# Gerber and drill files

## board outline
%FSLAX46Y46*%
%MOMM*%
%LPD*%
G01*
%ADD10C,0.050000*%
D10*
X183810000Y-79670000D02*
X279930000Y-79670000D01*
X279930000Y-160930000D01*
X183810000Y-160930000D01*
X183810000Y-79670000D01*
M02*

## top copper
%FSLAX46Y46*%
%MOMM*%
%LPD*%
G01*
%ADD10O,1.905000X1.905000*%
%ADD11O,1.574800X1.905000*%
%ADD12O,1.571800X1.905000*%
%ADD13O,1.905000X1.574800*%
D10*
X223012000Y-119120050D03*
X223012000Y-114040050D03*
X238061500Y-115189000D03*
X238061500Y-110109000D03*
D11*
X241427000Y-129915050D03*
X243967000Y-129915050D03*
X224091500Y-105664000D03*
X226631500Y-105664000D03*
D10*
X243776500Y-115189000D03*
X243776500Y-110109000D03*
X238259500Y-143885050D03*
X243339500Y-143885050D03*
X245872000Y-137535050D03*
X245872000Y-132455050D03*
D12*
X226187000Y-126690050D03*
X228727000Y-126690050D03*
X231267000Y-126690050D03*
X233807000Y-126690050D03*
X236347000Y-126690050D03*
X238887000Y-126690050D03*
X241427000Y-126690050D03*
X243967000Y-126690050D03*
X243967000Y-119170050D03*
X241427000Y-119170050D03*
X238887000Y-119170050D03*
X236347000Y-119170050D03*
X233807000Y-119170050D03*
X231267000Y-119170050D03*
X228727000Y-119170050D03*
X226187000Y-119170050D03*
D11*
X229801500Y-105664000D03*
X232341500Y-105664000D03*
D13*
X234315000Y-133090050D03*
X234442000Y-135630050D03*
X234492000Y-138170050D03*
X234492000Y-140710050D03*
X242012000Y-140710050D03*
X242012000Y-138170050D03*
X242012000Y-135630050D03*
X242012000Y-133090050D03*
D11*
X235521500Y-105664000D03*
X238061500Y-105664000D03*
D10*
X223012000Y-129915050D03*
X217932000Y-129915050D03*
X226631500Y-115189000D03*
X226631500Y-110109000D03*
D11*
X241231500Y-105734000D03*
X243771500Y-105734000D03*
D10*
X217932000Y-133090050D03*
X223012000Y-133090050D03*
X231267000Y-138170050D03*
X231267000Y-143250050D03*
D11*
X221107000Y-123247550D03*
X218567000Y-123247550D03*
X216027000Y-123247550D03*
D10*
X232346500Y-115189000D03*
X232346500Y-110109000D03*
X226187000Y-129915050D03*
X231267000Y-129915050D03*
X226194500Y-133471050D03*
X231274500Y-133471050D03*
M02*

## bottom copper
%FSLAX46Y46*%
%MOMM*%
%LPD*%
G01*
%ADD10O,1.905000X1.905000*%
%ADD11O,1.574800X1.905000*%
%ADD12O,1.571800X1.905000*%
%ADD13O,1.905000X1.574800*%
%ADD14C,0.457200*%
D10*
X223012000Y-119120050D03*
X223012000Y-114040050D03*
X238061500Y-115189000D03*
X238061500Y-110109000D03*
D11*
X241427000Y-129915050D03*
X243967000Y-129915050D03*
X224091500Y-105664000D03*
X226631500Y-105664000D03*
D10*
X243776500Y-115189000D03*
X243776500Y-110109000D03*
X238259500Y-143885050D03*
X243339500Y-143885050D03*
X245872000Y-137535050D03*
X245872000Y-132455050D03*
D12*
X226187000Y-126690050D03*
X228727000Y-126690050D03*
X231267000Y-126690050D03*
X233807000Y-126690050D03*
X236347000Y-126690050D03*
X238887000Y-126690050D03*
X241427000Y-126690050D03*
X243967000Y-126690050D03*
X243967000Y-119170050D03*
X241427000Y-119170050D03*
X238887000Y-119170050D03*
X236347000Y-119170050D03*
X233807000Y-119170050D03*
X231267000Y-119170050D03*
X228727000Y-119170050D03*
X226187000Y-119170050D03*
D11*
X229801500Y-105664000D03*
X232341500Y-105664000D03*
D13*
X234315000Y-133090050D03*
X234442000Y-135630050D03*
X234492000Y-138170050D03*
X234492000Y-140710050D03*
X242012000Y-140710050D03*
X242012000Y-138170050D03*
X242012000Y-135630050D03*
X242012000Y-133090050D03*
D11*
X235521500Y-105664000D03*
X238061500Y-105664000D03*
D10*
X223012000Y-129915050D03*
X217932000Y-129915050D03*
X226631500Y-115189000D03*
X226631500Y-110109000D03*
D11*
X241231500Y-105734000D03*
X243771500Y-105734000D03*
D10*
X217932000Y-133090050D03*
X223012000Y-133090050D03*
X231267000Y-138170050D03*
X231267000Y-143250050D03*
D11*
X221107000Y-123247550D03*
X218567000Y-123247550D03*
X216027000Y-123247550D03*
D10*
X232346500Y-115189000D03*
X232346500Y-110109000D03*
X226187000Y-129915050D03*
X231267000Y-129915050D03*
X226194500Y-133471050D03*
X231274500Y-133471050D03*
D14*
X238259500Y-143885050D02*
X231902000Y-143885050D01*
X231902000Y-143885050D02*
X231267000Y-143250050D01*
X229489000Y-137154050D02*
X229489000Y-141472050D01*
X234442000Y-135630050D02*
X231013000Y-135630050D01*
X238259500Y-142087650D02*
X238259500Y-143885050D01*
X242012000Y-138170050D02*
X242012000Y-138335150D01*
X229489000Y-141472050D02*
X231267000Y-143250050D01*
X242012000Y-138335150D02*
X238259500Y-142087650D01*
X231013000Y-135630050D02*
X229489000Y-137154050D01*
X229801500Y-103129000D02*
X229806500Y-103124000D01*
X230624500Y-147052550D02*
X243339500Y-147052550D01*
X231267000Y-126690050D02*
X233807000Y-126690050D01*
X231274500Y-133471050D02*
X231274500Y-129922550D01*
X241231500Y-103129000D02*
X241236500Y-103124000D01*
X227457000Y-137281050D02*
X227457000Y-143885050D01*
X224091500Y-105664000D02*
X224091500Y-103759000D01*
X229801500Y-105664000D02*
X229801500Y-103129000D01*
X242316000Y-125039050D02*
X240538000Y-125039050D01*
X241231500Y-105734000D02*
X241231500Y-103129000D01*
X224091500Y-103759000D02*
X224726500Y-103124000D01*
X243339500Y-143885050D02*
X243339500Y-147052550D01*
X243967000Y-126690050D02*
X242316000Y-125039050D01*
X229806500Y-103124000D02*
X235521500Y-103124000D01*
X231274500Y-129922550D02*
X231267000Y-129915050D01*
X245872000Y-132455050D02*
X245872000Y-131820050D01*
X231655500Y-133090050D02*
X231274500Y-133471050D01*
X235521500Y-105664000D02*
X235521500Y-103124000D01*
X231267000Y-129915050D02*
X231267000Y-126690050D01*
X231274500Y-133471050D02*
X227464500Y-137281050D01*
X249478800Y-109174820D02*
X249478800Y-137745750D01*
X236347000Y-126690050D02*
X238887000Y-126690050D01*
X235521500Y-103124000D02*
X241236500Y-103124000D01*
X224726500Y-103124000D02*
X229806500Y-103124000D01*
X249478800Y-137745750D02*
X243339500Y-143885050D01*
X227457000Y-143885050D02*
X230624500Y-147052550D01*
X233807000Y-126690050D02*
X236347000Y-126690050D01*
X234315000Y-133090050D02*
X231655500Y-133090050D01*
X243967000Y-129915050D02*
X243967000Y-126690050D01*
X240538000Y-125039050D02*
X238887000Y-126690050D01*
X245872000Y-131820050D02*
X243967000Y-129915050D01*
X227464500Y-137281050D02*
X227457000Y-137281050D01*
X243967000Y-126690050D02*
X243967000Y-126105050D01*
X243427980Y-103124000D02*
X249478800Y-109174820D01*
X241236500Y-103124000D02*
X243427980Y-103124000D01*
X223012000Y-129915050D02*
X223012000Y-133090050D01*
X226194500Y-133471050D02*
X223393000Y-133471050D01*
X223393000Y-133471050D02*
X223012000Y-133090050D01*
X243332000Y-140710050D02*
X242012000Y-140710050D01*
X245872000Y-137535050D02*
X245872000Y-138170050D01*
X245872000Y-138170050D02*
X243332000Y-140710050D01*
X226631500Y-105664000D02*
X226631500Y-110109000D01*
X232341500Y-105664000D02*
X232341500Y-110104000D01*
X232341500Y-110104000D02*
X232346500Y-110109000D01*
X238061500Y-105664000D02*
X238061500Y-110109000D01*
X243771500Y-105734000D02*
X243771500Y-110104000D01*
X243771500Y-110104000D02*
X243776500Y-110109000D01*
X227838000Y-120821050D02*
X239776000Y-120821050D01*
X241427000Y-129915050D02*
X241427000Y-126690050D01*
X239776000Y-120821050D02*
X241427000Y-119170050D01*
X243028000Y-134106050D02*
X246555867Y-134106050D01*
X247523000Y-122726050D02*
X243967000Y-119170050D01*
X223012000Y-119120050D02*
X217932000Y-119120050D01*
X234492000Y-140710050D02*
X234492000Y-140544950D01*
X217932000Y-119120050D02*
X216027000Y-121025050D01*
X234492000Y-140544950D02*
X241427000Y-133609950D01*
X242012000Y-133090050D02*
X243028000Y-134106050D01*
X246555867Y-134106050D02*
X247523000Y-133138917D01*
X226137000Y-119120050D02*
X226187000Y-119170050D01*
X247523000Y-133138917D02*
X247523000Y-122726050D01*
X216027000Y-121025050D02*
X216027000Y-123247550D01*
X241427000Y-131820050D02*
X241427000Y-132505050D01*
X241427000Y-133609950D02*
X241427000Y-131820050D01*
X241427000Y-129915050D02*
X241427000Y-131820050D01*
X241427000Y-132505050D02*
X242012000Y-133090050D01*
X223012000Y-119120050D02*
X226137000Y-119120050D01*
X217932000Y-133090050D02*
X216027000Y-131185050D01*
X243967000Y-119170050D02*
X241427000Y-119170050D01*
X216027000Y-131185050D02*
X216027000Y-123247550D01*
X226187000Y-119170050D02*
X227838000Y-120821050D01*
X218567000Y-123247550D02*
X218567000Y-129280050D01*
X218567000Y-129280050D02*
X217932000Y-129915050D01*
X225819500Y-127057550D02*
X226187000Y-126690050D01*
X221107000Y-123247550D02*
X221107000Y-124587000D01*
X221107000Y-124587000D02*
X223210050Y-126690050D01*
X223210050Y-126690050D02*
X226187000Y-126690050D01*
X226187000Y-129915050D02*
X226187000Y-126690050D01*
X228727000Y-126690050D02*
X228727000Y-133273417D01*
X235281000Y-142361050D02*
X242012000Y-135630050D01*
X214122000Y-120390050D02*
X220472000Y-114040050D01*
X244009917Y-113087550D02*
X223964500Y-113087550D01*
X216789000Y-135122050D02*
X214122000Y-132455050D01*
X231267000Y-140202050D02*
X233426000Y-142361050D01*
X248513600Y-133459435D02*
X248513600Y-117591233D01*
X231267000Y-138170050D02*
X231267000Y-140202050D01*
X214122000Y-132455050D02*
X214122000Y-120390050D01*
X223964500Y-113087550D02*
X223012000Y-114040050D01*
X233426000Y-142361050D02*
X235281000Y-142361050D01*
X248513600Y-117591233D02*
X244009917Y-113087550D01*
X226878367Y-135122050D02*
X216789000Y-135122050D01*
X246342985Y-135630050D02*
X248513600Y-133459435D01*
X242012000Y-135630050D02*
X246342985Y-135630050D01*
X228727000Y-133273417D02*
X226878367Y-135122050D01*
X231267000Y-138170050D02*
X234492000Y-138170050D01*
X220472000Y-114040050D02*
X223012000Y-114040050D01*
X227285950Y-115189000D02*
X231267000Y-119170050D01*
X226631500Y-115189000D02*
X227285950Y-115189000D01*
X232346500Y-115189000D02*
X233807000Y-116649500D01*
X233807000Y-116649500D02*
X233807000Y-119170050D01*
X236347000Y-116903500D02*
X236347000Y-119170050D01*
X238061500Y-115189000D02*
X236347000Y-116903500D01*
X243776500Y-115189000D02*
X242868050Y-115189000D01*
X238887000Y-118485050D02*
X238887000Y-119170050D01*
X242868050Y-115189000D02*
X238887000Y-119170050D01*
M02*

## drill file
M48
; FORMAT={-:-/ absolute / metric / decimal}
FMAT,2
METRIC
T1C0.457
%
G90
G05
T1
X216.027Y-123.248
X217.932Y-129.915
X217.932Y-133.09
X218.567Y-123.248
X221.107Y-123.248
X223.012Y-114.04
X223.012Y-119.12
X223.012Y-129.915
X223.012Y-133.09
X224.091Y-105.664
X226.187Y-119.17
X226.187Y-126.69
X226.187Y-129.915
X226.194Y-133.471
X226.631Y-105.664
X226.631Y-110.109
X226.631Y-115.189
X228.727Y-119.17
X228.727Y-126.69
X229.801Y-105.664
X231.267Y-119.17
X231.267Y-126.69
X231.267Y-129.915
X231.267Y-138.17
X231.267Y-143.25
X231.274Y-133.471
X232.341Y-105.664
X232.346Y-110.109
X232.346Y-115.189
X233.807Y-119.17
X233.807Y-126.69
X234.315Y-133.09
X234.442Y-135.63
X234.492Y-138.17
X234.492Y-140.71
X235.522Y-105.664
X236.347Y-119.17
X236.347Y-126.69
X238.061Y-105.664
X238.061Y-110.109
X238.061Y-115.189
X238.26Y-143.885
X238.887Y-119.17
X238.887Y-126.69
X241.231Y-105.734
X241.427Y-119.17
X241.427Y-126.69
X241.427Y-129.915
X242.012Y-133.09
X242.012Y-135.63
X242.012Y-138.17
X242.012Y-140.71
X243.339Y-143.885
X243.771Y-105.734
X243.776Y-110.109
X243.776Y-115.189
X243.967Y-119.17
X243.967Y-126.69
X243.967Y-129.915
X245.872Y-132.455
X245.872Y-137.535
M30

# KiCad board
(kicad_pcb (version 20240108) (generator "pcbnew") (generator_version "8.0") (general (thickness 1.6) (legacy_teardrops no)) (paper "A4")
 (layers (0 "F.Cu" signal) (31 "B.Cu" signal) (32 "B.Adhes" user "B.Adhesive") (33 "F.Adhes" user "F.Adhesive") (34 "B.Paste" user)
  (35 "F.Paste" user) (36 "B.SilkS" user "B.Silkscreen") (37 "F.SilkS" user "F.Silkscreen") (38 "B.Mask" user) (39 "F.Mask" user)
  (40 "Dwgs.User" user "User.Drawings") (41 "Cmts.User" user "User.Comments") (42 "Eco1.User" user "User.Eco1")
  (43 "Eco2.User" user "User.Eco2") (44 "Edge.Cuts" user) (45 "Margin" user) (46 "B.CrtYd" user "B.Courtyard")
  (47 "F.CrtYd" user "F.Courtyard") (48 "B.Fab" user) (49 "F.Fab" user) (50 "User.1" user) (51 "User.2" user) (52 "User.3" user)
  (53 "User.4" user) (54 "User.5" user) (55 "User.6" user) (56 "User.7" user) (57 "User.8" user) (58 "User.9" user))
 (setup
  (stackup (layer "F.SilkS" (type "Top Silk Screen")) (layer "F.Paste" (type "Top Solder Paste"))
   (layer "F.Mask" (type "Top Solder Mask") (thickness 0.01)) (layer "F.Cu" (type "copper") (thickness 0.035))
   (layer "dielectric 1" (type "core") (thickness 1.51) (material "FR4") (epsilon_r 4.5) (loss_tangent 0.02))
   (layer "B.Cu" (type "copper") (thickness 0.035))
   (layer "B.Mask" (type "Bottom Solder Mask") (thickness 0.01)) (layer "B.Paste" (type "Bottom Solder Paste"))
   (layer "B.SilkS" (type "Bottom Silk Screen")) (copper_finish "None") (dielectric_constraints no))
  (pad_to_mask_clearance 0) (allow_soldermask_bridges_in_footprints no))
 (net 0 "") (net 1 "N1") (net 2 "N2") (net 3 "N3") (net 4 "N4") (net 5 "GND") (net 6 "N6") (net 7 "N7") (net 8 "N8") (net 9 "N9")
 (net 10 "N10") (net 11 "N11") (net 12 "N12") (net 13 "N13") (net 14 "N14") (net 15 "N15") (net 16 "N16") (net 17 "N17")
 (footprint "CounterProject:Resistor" (layer "F.Cu") (at 223.012 119.12005 90)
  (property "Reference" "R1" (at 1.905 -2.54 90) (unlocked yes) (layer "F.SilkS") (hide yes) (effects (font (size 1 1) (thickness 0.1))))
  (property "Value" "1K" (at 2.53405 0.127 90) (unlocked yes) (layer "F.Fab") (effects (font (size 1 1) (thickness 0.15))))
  (pad "1" thru_hole oval (at 0 0 90) (size 1.905 1.905) (drill 0.4572) (layers "*.Cu" "*.Mask") (remove_unused_layers no) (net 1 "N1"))
  (pad "2" thru_hole oval (at 5.08 0 90) (size 1.905 1.905) (drill 0.4572) (layers "*.Cu" "*.Mask") (remove_unused_layers no) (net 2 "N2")))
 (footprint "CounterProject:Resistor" (layer "F.Cu") (at 238.0615 115.189 90)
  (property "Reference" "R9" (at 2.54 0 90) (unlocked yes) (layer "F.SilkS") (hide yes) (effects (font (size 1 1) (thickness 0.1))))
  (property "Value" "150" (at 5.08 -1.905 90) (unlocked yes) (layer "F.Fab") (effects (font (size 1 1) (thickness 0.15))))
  (pad "1" thru_hole oval (at 0 0 90) (size 1.905 1.905) (drill 0.4572) (layers "*.Cu" "*.Mask") (remove_unused_layers no) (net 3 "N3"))
  (pad "2" thru_hole oval (at 5.08 0 90) (size 1.905 1.905) (drill 0.4572) (layers "*.Cu" "*.Mask") (remove_unused_layers no) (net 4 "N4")))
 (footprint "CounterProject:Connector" (layer "F.Cu") (at 241.427 129.91505)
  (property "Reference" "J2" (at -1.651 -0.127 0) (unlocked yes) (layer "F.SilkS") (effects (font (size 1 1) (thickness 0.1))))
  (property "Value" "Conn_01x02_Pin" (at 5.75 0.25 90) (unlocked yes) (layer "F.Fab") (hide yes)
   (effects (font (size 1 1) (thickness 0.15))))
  (pad "1" thru_hole oval (at 0 0) (size 1.5748 1.905) (drill 0.4572) (layers "*.Cu" "*.Mask") (remove_unused_layers no) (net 1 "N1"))
  (pad "2" thru_hole oval (at 2.54 0) (size 1.5748 1.905) (drill 0.4572) (layers "*.Cu" "*.Mask") (remove_unused_layers no) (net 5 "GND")))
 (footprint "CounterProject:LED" (layer "F.Cu") (at 224.0915 105.664)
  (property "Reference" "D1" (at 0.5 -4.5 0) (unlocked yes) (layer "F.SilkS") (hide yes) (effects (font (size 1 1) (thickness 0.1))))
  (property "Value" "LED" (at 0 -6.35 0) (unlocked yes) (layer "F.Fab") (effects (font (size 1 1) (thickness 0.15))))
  (pad "1" thru_hole oval (at 0 0) (size 1.5748 1.905) (drill 0.4572) (layers "*.Cu" "*.Mask") (remove_unused_layers no) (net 5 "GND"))
  (pad "2" thru_hole oval (at 2.54 0) (size 1.5748 1.905) (drill 0.4572) (layers "*.Cu" "*.Mask") (remove_unused_layers no) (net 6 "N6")))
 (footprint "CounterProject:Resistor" (layer "F.Cu") (at 243.7765 115.189 90)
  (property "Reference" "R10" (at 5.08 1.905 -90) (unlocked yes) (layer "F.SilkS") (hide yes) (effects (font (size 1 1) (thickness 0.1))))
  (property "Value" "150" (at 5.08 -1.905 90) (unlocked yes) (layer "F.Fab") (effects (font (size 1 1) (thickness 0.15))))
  (pad "1" thru_hole oval (at 0 0 90) (size 1.905 1.905) (drill 0.4572) (layers "*.Cu" "*.Mask") (remove_unused_layers no) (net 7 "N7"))
  (pad "2" thru_hole oval (at 5.08 0 90) (size 1.905 1.905) (drill 0.4572) (layers "*.Cu" "*.Mask") (remove_unused_layers no) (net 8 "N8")))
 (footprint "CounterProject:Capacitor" (layer "F.Cu") (at 238.2595 143.88505)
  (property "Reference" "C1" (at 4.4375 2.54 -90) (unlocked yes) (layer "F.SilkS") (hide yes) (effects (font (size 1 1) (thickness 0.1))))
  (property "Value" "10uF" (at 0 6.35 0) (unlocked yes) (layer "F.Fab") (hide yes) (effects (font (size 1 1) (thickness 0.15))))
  (pad "1" thru_hole oval (at 0 0) (size 1.905 1.905) (drill 0.4572) (layers "*.Cu" "*.Mask") (remove_unused_layers no) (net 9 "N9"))
  (pad "2" thru_hole oval (at 5.08 0) (size 1.905 1.905) (drill 0.4572) (layers "*.Cu" "*.Mask") (remove_unused_layers no) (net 5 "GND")))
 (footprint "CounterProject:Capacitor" (layer "F.Cu") (at 245.872 137.53505 90)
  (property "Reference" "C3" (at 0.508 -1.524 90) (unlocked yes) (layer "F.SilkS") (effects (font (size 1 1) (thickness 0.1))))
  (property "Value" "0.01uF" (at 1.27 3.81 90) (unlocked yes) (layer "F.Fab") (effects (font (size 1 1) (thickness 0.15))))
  (pad "1" thru_hole oval (at 0 0 90) (size 1.905 1.905) (drill 0.4572) (layers "*.Cu" "*.Mask") (remove_unused_layers no) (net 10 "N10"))
  (pad "2" thru_hole oval (at 5.08 0 90) (size 1.905 1.905) (drill 0.4572) (layers "*.Cu" "*.Mask") (remove_unused_layers no) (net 5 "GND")))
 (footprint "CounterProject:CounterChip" (layer "F.Cu") (at 226.1616 126.66465)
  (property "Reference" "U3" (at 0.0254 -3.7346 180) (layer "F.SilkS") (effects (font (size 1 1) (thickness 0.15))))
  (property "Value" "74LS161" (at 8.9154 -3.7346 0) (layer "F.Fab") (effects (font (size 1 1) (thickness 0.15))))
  (pad "1" thru_hole oval (at 0.0254 0.0254) (size 1.5718 1.905) (drill 0.4572) (layers "*.Cu" "*.Mask") (remove_unused_layers no)
   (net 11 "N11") (thermal_bridge_angle 45))
  (pad "2" thru_hole oval (at 2.5654 0.0254) (size 1.5718 1.905) (drill 0.4572) (layers "*.Cu" "*.Mask") (remove_unused_layers no)
   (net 2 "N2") (thermal_bridge_angle 45))
  (pad "3" thru_hole oval (at 5.1054 0.0254) (size 1.5718 1.905) (drill 0.4572) (layers "*.Cu" "*.Mask") (remove_unused_layers no)
   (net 5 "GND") (thermal_bridge_angle 45))
  (pad "4" thru_hole oval (at 7.6454 0.0254) (size 1.5718 1.905) (drill 0.4572) (layers "*.Cu" "*.Mask") (remove_unused_layers no)
   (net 5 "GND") (thermal_bridge_angle 45))
  (pad "5" thru_hole oval (at 10.1854 0.0254) (size 1.5718 1.905) (drill 0.4572) (layers "*.Cu" "*.Mask") (remove_unused_layers no)
   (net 5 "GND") (thermal_bridge_angle 45))
  (pad "6" thru_hole oval (at 12.7254 0.0254) (size 1.5718 1.905) (drill 0.4572) (layers "*.Cu" "*.Mask") (remove_unused_layers no)
   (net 5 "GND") (thermal_bridge_angle 45))
  (pad "7" thru_hole oval (at 15.2654 0.0254) (size 1.5718 1.905) (drill 0.4572) (layers "*.Cu" "*.Mask") (remove_unused_layers no)
   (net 1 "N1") (thermal_bridge_angle 45))
  (pad "8" thru_hole oval (at 17.8054 0.0254) (size 1.5718 1.905) (drill 0.4572) (layers "*.Cu" "*.Mask") (remove_unused_layers no)
   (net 5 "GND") (thermal_bridge_angle 45))
  (pad "9" thru_hole oval (at 17.8054 -7.4946) (size 1.5718 1.905) (drill 0.4572) (layers "*.Cu" "*.Mask") (remove_unused_layers no)
   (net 1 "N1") (thermal_bridge_angle 45))
  (pad "10" thru_hole oval (at 15.2654 -7.4946) (size 1.5718 1.905) (drill 0.4572) (layers "*.Cu" "*.Mask") (remove_unused_layers no)
   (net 1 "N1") (thermal_bridge_angle 45))
  (pad "11" thru_hole oval (at 12.7254 -7.4946) (size 1.5718 1.905) (drill 0.4572) (layers "*.Cu" "*.Mask") (remove_unused_layers no)
   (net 7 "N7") (thermal_bridge_angle 45))
  (pad "12" thru_hole oval (at 10.1854 -7.4946) (size 1.5718 1.905) (drill 0.4572) (layers "*.Cu" "*.Mask") (remove_unused_layers no)
   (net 3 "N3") (thermal_bridge_angle 45))
  (pad "13" thru_hole oval (at 7.6454 -7.4946) (size 1.5718 1.905) (drill 0.4572) (layers "*.Cu" "*.Mask") (remove_unused_layers no)
   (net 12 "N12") (thermal_bridge_angle 45))
  (pad "14" thru_hole oval (at 5.1054 -7.4946) (size 1.5718 1.905) (drill 0.4572) (layers "*.Cu" "*.Mask") (remove_unused_layers no)
   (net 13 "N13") (thermal_bridge_angle 45))
  (pad "15" thru_hole oval (at 2.5654 -7.4946) (size 1.5718 1.905) (drill 0.4572) (layers "*.Cu" "*.Mask") (remove_unused_layers no)
   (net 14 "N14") (thermal_bridge_angle 45))
  (pad "16" thru_hole oval (at 0.0254 -7.4946) (size 1.5718 1.905) (drill 0.4572) (layers "*.Cu" "*.Mask") (remove_unused_layers no)
   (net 1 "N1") (thermal_bridge_angle 45)))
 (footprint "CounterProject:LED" (layer "F.Cu") (at 229.8015 105.664)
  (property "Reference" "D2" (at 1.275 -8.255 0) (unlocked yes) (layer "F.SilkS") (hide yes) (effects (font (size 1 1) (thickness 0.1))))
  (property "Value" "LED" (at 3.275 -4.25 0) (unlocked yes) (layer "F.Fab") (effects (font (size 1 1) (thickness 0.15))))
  (pad "1" thru_hole oval (at 0 0) (size 1.5748 1.905) (drill 0.4572) (layers "*.Cu" "*.Mask") (remove_unused_layers no) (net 5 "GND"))
  (pad "2" thru_hole oval (at 2.54 0) (size 1.5748 1.905) (drill 0.4572) (layers "*.Cu" "*.Mask") (remove_unused_layers no) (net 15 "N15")))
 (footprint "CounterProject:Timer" (layer "F.Cu") (at 234.315 133.09005 -90)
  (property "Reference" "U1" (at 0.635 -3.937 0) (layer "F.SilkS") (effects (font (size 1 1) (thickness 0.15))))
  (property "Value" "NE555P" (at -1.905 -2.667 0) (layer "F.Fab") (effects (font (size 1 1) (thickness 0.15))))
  (pad "1" thru_hole oval (at 0 0 270) (size 1.5748 1.905) (drill 0.4572) (layers "*.Cu" "*.Mask") (remove_unused_layers no) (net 5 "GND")
   (thermal_bridge_angle 45))
  (pad "2" thru_hole oval (at 2.54 -0.127 270) (size 1.5748 1.905) (drill 0.4572) (layers "*.Cu" "*.Mask") (remove_unused_layers no)
   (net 9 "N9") (thermal_bridge_angle 45))
  (pad "3" thru_hole oval (at 5.08 -0.177 270) (size 1.5748 1.905) (drill 0.4572) (layers "*.Cu" "*.Mask") (remove_unused_layers no)
   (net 2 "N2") (thermal_bridge_angle 45))
  (pad "4" thru_hole oval (at 7.62 -0.177 270) (size 1.5748 1.905) (drill 0.4572) (layers "*.Cu" "*.Mask") (remove_unused_layers no)
   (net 1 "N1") (thermal_bridge_angle 45))
  (pad "5" thru_hole oval (at 7.62 -7.697 270) (size 1.5748 1.905) (drill 0.4572) (layers "*.Cu" "*.Mask") (remove_unused_layers no)
   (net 10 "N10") (thermal_bridge_angle 45))
  (pad "6" thru_hole oval (at 5.08 -7.697 270) (size 1.5748 1.905) (drill 0.4572) (layers "*.Cu" "*.Mask") (remove_unused_layers no)
   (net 9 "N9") (thermal_bridge_angle 45))
  (pad "7" thru_hole oval (at 2.54 -7.697 270) (size 1.5748 1.905) (drill 0.4572) (layers "*.Cu" "*.Mask") (remove_unused_layers no)
   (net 2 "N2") (thermal_bridge_angle 45))
  (pad "8" thru_hole oval (at 0 -7.697 270) (size 1.5748 1.905) (drill 0.4572) (layers "*.Cu" "*.Mask") (remove_unused_layers no)
   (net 1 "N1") (thermal_bridge_angle 45)))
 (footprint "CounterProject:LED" (layer "F.Cu") (at 235.5215 105.664)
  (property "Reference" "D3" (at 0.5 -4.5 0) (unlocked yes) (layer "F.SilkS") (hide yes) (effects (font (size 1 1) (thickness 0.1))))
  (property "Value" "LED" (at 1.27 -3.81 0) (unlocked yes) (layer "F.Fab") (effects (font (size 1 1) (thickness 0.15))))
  (pad "1" thru_hole oval (at 0 0) (size 1.5748 1.905) (drill 0.4572) (layers "*.Cu" "*.Mask") (remove_unused_layers no) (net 5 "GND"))
  (pad "2" thru_hole oval (at 2.54 0) (size 1.5748 1.905) (drill 0.4572) (layers "*.Cu" "*.Mask") (remove_unused_layers no) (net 4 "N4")))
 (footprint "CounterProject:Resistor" (layer "F.Cu") (at 223.012 129.91505 180)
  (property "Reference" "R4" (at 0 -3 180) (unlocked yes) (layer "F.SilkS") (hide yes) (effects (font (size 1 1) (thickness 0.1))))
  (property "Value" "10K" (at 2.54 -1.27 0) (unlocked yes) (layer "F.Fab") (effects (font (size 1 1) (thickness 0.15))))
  (pad "1" thru_hole oval (at 0 0 180) (size 1.905 1.905) (drill 0.4572) (layers "*.Cu" "*.Mask") (remove_unused_layers no) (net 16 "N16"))
  (pad "2" thru_hole oval (at 5.08 0 180) (size 1.905 1.905) (drill 0.4572) (layers "*.Cu" "*.Mask") (remove_unused_layers no)
   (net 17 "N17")))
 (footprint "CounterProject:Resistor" (layer "F.Cu") (at 226.6315 115.189 90)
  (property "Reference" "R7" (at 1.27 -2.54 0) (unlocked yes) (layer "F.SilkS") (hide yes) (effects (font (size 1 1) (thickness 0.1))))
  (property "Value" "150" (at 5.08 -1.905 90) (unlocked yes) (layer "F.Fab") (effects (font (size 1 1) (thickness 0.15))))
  (pad "1" thru_hole oval (at 0 0 90) (size 1.905 1.905) (drill 0.4572) (layers "*.Cu" "*.Mask") (remove_unused_layers no) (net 13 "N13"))
  (pad "2" thru_hole oval (at 5.08 0 90) (size 1.905 1.905) (drill 0.4572) (layers "*.Cu" "*.Mask") (remove_unused_layers no) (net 6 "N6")))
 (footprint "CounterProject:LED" (layer "F.Cu") (at 241.2315 105.734)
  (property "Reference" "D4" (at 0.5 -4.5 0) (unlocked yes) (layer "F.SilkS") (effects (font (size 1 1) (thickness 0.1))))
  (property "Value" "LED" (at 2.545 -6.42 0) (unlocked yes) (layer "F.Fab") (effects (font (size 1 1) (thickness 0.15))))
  (pad "1" thru_hole oval (at 0 0) (size 1.5748 1.905) (drill 0.4572) (layers "*.Cu" "*.Mask") (remove_unused_layers no) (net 5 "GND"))
  (pad "2" thru_hole oval (at 2.54 0) (size 1.5748 1.905) (drill 0.4572) (layers "*.Cu" "*.Mask") (remove_unused_layers no) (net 8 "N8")))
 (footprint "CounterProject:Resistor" (layer "F.Cu") (at 217.932 133.09005)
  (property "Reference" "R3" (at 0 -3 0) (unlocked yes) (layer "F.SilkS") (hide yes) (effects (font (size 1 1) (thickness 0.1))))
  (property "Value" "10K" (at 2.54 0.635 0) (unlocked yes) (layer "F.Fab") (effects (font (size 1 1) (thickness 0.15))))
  (pad "1" thru_hole oval (at 0 0) (size 1.905 1.905) (drill 0.4572) (layers "*.Cu" "*.Mask") (remove_unused_layers no) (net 1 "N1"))
  (pad "2" thru_hole oval (at 5.08 0) (size 1.905 1.905) (drill 0.4572) (layers "*.Cu" "*.Mask") (remove_unused_layers no) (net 16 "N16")))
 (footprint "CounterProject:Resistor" (layer "F.Cu") (at 231.267 138.17005 -90)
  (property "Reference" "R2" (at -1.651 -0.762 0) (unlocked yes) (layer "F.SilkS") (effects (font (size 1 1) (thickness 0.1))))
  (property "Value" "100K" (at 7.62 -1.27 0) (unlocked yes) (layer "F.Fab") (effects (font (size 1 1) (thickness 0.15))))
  (pad "1" thru_hole oval (at 0 0 270) (size 1.905 1.905) (drill 0.4572) (layers "*.Cu" "*.Mask") (remove_unused_layers no) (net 2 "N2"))
  (pad "2" thru_hole oval (at 5.08 0 270) (size 1.905 1.905) (drill 0.4572) (layers "*.Cu" "*.Mask") (remove_unused_layers no) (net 9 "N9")))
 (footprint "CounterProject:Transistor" (layer "F.Cu") (at 221.107 123.24755 180)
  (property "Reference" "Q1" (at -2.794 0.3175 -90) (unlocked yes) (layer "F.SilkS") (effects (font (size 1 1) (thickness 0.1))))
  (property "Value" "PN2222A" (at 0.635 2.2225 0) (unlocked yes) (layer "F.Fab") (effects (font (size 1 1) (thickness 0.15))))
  (pad "1" thru_hole oval (at 0 0 180) (size 1.5748 1.905) (drill 0.4572) (layers "*.Cu" "*.Mask") (remove_unused_layers no) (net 11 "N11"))
  (pad "2" thru_hole oval (at 2.54 0 180) (size 1.5748 1.905) (drill 0.4572) (layers "*.Cu" "*.Mask") (remove_unused_layers no)
   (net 17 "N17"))
  (pad "3" thru_hole oval (at 5.08 0 180) (size 1.5748 1.905) (drill 0.4572) (layers "*.Cu" "*.Mask") (remove_unused_layers no) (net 1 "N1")))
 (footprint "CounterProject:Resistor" (layer "F.Cu") (at 232.3465 115.189 90)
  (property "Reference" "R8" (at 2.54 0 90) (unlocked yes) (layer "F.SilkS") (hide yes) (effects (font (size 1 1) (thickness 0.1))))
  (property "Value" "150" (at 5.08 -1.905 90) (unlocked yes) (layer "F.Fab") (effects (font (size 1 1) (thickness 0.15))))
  (pad "1" thru_hole oval (at 0 0 90) (size 1.905 1.905) (drill 0.4572) (layers "*.Cu" "*.Mask") (remove_unused_layers no) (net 12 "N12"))
  (pad "2" thru_hole oval (at 5.08 0 90) (size 1.905 1.905) (drill 0.4572) (layers "*.Cu" "*.Mask") (remove_unused_layers no) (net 15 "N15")))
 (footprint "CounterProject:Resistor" (layer "F.Cu") (at 226.187 129.91505)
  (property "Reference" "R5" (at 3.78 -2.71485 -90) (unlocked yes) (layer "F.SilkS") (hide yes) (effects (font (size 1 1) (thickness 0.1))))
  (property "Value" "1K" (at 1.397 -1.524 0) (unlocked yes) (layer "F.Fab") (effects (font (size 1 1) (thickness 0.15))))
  (pad "1" thru_hole oval (at 0 0) (size 1.905 1.905) (drill 0.4572) (layers "*.Cu" "*.Mask") (remove_unused_layers no) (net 11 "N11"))
  (pad "2" thru_hole oval (at 5.08 0) (size 1.905 1.905) (drill 0.4572) (layers "*.Cu" "*.Mask") (remove_unused_layers no) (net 5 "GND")))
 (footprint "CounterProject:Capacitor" (layer "F.Cu") (at 226.1945 133.47105)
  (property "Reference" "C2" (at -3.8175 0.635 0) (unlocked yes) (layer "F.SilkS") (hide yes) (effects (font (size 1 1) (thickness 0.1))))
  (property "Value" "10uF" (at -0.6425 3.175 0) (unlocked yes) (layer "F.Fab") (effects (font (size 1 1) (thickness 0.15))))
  (pad "1" thru_hole oval (at 0 0) (size 1.905 1.905) (drill 0.4572) (layers "*.Cu" "*.Mask") (remove_unused_layers no) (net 16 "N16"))
  (pad "2" thru_hole oval (at 5.08 0) (size 1.905 1.905) (drill 0.4572) (layers "*.Cu" "*.Mask") (remove_unused_layers no) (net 5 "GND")))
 (gr_rect (start 183.81 79.67) (end 279.93 160.93) (stroke (width 0.05) (type default)) (fill none) (layer "Edge.Cuts"))
 (segment (start 238.2595 143.88505) (end 231.902 143.88505) (width 0.4572) (layer "B.Cu") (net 9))
 (segment (start 231.902 143.88505) (end 231.267 143.25005) (width 0.4572) (layer "B.Cu") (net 9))
 (segment (start 229.489 137.15405) (end 229.489 141.47205) (width 0.4572) (layer "B.Cu") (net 9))
 (segment (start 234.442 135.63005) (end 231.013 135.63005) (width 0.4572) (layer "B.Cu") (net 9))
 (segment (start 238.2595 142.08765) (end 238.2595 143.88505) (width 0.4572) (layer "B.Cu") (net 9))
 (segment (start 242.012 138.17005) (end 242.012 138.33515) (width 0.4572) (layer "B.Cu") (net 9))
 (segment (start 229.489 141.47205) (end 231.267 143.25005) (width 0.4572) (layer "B.Cu") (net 9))
 (segment (start 242.012 138.33515) (end 238.2595 142.08765) (width 0.4572) (layer "B.Cu") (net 9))
 (segment (start 231.013 135.63005) (end 229.489 137.15405) (width 0.4572) (layer "B.Cu") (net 9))
 (segment (start 229.8015 103.129) (end 229.8065 103.124) (width 0.4572) (layer "B.Cu") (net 5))
 (segment (start 230.6245 147.05255) (end 243.3395 147.05255) (width 0.4572) (layer "B.Cu") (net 5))
 (segment (start 231.267 126.69005) (end 233.807 126.69005) (width 0.4572) (layer "B.Cu") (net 5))
 (segment (start 231.2745 133.47105) (end 231.2745 129.92255) (width 0.4572) (layer "B.Cu") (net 5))
 (segment (start 241.2315 103.129) (end 241.2365 103.124) (width 0.4572) (layer "B.Cu") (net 5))
 (segment (start 227.457 137.28105) (end 227.457 143.88505) (width 0.4572) (layer "B.Cu") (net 5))
 (segment (start 224.0915 105.664) (end 224.0915 103.759) (width 0.4572) (layer "B.Cu") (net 5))
 (segment (start 229.8015 105.664) (end 229.8015 103.129) (width 0.4572) (layer "B.Cu") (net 5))
 (segment (start 242.316 125.03905) (end 240.538 125.03905) (width 0.4572) (layer "B.Cu") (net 5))
 (segment (start 241.2315 105.734) (end 241.2315 103.129) (width 0.4572) (layer "B.Cu") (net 5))
 (segment (start 224.0915 103.759) (end 224.7265 103.124) (width 0.4572) (layer "B.Cu") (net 5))
 (segment (start 243.3395 143.88505) (end 243.3395 147.05255) (width 0.4572) (layer "B.Cu") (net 5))
 (segment (start 243.967 126.69005) (end 242.316 125.03905) (width 0.4572) (layer "B.Cu") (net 5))
 (segment (start 229.8065 103.124) (end 235.5215 103.124) (width 0.4572) (layer "B.Cu") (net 5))
 (segment (start 231.2745 129.92255) (end 231.267 129.91505) (width 0.4572) (layer "B.Cu") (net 5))
 (segment (start 245.872 132.45505) (end 245.872 131.82005) (width 0.4572) (layer "B.Cu") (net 5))
 (segment (start 231.6555 133.09005) (end 231.2745 133.47105) (width 0.4572) (layer "B.Cu") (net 5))
 (segment (start 235.5215 105.664) (end 235.5215 103.124) (width 0.4572) (layer "B.Cu") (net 5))
 (segment (start 231.267 129.91505) (end 231.267 126.69005) (width 0.4572) (layer "B.Cu") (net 5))
 (segment (start 231.2745 133.47105) (end 227.4645 137.28105) (width 0.4572) (layer "B.Cu") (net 5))
 (segment (start 249.4788 109.17482) (end 249.4788 137.74575) (width 0.4572) (layer "B.Cu") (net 5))
 (segment (start 236.347 126.69005) (end 238.887 126.69005) (width 0.4572) (layer "B.Cu") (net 5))
 (segment (start 235.5215 103.124) (end 241.2365 103.124) (width 0.4572) (layer "B.Cu") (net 5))
 (segment (start 224.7265 103.124) (end 229.8065 103.124) (width 0.4572) (layer "B.Cu") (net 5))
 (segment (start 249.4788 137.74575) (end 243.3395 143.88505) (width 0.4572) (layer "B.Cu") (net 5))
 (segment (start 227.457 143.88505) (end 230.6245 147.05255) (width 0.4572) (layer "B.Cu") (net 5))
 (segment (start 233.807 126.69005) (end 236.347 126.69005) (width 0.4572) (layer "B.Cu") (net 5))
 (segment (start 234.315 133.09005) (end 231.6555 133.09005) (width 0.4572) (layer "B.Cu") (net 5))
 (segment (start 243.967 129.91505) (end 243.967 126.69005) (width 0.4572) (layer "B.Cu") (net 5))
 (segment (start 240.538 125.03905) (end 238.887 126.69005) (width 0.4572) (layer "B.Cu") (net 5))
 (segment (start 245.872 131.82005) (end 243.967 129.91505) (width 0.4572) (layer "B.Cu") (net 5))
 (segment (start 227.4645 137.28105) (end 227.457 137.28105) (width 0.4572) (layer "B.Cu") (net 5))
 (segment (start 243.967 126.69005) (end 243.967 126.10505) (width 0.4572) (layer "B.Cu") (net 5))
 (segment (start 243.42798 103.124) (end 249.4788 109.17482) (width 0.4572) (layer "B.Cu") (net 5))
 (segment (start 241.2365 103.124) (end 243.42798 103.124) (width 0.4572) (layer "B.Cu") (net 5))
 (segment (start 223.012 129.91505) (end 223.012 133.09005) (width 0.4572) (layer "B.Cu") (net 16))
 (segment (start 226.1945 133.47105) (end 223.393 133.47105) (width 0.4572) (layer "B.Cu") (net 16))
 (segment (start 223.393 133.47105) (end 223.012 133.09005) (width 0.4572) (layer "B.Cu") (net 16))
 (segment (start 243.332 140.71005) (end 242.012 140.71005) (width 0.4572) (layer "B.Cu") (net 10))
 (segment (start 245.872 137.53505) (end 245.872 138.17005) (width 0.4572) (layer "B.Cu") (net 10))
 (segment (start 245.872 138.17005) (end 243.332 140.71005) (width 0.4572) (layer "B.Cu") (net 10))
 (segment (start 226.6315 105.664) (end 226.6315 110.109) (width 0.4572) (layer "B.Cu") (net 6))
 (segment (start 232.3415 105.664) (end 232.3415 110.104) (width 0.4572) (layer "B.Cu") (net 15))
 (segment (start 232.3415 110.104) (end 232.3465 110.109) (width 0.4572) (layer "B.Cu") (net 15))
 (segment (start 238.0615 105.664) (end 238.0615 110.109) (width 0.4572) (layer "B.Cu") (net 4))
 (segment (start 243.7715 105.734) (end 243.7715 110.104) (width 0.4572) (layer "B.Cu") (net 8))
 (segment (start 243.7715 110.104) (end 243.7765 110.109) (width 0.4572) (layer "B.Cu") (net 8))
 (segment (start 227.838 120.82105) (end 239.776 120.82105) (width 0.4572) (layer "B.Cu") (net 1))
 (segment (start 241.427 129.91505) (end 241.427 126.69005) (width 0.4572) (layer "B.Cu") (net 1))
 (segment (start 239.776 120.82105) (end 241.427 119.17005) (width 0.4572) (layer "B.Cu") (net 1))
 (segment (start 243.028 134.10605) (end 246.555867 134.10605) (width 0.4572) (layer "B.Cu") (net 1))
 (segment (start 247.523 122.72605) (end 243.967 119.17005) (width 0.4572) (layer "B.Cu") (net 1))
 (segment (start 223.012 119.12005) (end 217.932 119.12005) (width 0.4572) (layer "B.Cu") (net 1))
 (segment (start 234.492 140.71005) (end 234.492 140.54495) (width 0.4572) (layer "B.Cu") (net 1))
 (segment (start 217.932 119.12005) (end 216.027 121.02505) (width 0.4572) (layer "B.Cu") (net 1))
 (segment (start 234.492 140.54495) (end 241.427 133.60995) (width 0.4572) (layer "B.Cu") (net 1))
 (segment (start 242.012 133.09005) (end 243.028 134.10605) (width 0.4572) (layer "B.Cu") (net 1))
 (segment (start 246.555867 134.10605) (end 247.523 133.138917) (width 0.4572) (layer "B.Cu") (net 1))
 (segment (start 226.137 119.12005) (end 226.187 119.17005) (width 0.4572) (layer "B.Cu") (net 1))
 (segment (start 247.523 133.138917) (end 247.523 122.72605) (width 0.4572) (layer "B.Cu") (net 1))
 (segment (start 216.027 121.02505) (end 216.027 123.24755) (width 0.4572) (layer "B.Cu") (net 1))
 (segment (start 241.427 131.82005) (end 241.427 132.50505) (width 0.4572) (layer "B.Cu") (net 1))
 (segment (start 241.427 133.60995) (end 241.427 131.82005) (width 0.4572) (layer "B.Cu") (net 1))
 (segment (start 241.427 129.91505) (end 241.427 131.82005) (width 0.4572) (layer "B.Cu") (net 1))
 (segment (start 241.427 132.50505) (end 242.012 133.09005) (width 0.4572) (layer "B.Cu") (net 1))
 (segment (start 223.012 119.12005) (end 226.137 119.12005) (width 0.4572) (layer "B.Cu") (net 1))
 (segment (start 217.932 133.09005) (end 216.027 131.18505) (width 0.4572) (layer "B.Cu") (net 1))
 (segment (start 243.967 119.17005) (end 241.427 119.17005) (width 0.4572) (layer "B.Cu") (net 1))
 (segment (start 216.027 131.18505) (end 216.027 123.24755) (width 0.4572) (layer "B.Cu") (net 1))
 (segment (start 226.187 119.17005) (end 227.838 120.82105) (width 0.4572) (layer "B.Cu") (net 1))
 (segment (start 218.567 123.24755) (end 218.567 129.28005) (width 0.4572) (layer "B.Cu") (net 17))
 (segment (start 218.567 129.28005) (end 217.932 129.91505) (width 0.4572) (layer "B.Cu") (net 17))
 (segment (start 225.8195 127.05755) (end 226.187 126.69005) (width 0.4572) (layer "B.Cu") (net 11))
 (segment (start 221.107 123.24755) (end 221.107 124.587) (width 0.4572) (layer "B.Cu") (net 11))
 (segment (start 221.107 124.587) (end 223.21005 126.69005) (width 0.4572) (layer "B.Cu") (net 11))
 (segment (start 223.21005 126.69005) (end 226.187 126.69005) (width 0.4572) (layer "B.Cu") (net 11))
 (segment (start 226.187 129.91505) (end 226.187 126.69005) (width 0.4572) (layer "B.Cu") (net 11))
 (segment (start 228.727 126.69005) (end 228.727 133.273417) (width 0.4572) (layer "B.Cu") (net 2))
 (segment (start 235.281 142.36105) (end 242.012 135.63005) (width 0.4572) (layer "B.Cu") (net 2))
 (segment (start 214.122 120.39005) (end 220.472 114.04005) (width 0.4572) (layer "B.Cu") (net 2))
 (segment (start 244.009917 113.08755) (end 223.9645 113.08755) (width 0.4572) (layer "B.Cu") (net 2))
 (segment (start 216.789 135.12205) (end 214.122 132.45505) (width 0.4572) (layer "B.Cu") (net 2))
 (segment (start 231.267 140.20205) (end 233.426 142.36105) (width 0.4572) (layer "B.Cu") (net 2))
 (segment (start 248.5136 133.459435) (end 248.5136 117.591233) (width 0.4572) (layer "B.Cu") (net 2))
 (segment (start 231.267 138.17005) (end 231.267 140.20205) (width 0.4572) (layer "B.Cu") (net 2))
 (segment (start 214.122 132.45505) (end 214.122 120.39005) (width 0.4572) (layer "B.Cu") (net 2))
 (segment (start 223.9645 113.08755) (end 223.012 114.04005) (width 0.4572) (layer "B.Cu") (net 2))
 (segment (start 233.426 142.36105) (end 235.281 142.36105) (width 0.4572) (layer "B.Cu") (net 2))
 (segment (start 248.5136 117.591233) (end 244.009917 113.08755) (width 0.4572) (layer "B.Cu") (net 2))
 (segment (start 226.878367 135.12205) (end 216.789 135.12205) (width 0.4572) (layer "B.Cu") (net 2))
 (segment (start 246.342985 135.63005) (end 248.5136 133.459435) (width 0.4572) (layer "B.Cu") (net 2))
 (segment (start 242.012 135.63005) (end 246.342985 135.63005) (width 0.4572) (layer "B.Cu") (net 2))
 (segment (start 228.727 133.273417) (end 226.878367 135.12205) (width 0.4572) (layer "B.Cu") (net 2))
 (segment (start 231.267 138.17005) (end 234.492 138.17005) (width 0.4572) (layer "B.Cu") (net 2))
 (segment (start 220.472 114.04005) (end 223.012 114.04005) (width 0.4572) (layer "B.Cu") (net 2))
 (segment (start 227.28595 115.189) (end 231.267 119.17005) (width 0.4572) (layer "B.Cu") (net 13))
 (segment (start 226.6315 115.189) (end 227.28595 115.189) (width 0.4572) (layer "B.Cu") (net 13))
 (segment (start 232.3465 115.189) (end 233.807 116.6495) (width 0.4572) (layer "B.Cu") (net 12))
 (segment (start 233.807 116.6495) (end 233.807 119.17005) (width 0.4572) (layer "B.Cu") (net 12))
 (segment (start 236.347 116.9035) (end 236.347 119.17005) (width 0.4572) (layer "B.Cu") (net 3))
 (segment (start 238.0615 115.189) (end 236.347 116.9035) (width 0.4572) (layer "B.Cu") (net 3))
 (segment (start 243.7765 115.189) (end 242.86805 115.189) (width 0.4572) (layer "B.Cu") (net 7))
 (segment (start 238.887 118.48505) (end 238.887 119.17005) (width 0.4572) (layer "B.Cu") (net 7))
 (segment (start 242.86805 115.189) (end 238.887 119.17005) (width 0.4572) (layer "B.Cu") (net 7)))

